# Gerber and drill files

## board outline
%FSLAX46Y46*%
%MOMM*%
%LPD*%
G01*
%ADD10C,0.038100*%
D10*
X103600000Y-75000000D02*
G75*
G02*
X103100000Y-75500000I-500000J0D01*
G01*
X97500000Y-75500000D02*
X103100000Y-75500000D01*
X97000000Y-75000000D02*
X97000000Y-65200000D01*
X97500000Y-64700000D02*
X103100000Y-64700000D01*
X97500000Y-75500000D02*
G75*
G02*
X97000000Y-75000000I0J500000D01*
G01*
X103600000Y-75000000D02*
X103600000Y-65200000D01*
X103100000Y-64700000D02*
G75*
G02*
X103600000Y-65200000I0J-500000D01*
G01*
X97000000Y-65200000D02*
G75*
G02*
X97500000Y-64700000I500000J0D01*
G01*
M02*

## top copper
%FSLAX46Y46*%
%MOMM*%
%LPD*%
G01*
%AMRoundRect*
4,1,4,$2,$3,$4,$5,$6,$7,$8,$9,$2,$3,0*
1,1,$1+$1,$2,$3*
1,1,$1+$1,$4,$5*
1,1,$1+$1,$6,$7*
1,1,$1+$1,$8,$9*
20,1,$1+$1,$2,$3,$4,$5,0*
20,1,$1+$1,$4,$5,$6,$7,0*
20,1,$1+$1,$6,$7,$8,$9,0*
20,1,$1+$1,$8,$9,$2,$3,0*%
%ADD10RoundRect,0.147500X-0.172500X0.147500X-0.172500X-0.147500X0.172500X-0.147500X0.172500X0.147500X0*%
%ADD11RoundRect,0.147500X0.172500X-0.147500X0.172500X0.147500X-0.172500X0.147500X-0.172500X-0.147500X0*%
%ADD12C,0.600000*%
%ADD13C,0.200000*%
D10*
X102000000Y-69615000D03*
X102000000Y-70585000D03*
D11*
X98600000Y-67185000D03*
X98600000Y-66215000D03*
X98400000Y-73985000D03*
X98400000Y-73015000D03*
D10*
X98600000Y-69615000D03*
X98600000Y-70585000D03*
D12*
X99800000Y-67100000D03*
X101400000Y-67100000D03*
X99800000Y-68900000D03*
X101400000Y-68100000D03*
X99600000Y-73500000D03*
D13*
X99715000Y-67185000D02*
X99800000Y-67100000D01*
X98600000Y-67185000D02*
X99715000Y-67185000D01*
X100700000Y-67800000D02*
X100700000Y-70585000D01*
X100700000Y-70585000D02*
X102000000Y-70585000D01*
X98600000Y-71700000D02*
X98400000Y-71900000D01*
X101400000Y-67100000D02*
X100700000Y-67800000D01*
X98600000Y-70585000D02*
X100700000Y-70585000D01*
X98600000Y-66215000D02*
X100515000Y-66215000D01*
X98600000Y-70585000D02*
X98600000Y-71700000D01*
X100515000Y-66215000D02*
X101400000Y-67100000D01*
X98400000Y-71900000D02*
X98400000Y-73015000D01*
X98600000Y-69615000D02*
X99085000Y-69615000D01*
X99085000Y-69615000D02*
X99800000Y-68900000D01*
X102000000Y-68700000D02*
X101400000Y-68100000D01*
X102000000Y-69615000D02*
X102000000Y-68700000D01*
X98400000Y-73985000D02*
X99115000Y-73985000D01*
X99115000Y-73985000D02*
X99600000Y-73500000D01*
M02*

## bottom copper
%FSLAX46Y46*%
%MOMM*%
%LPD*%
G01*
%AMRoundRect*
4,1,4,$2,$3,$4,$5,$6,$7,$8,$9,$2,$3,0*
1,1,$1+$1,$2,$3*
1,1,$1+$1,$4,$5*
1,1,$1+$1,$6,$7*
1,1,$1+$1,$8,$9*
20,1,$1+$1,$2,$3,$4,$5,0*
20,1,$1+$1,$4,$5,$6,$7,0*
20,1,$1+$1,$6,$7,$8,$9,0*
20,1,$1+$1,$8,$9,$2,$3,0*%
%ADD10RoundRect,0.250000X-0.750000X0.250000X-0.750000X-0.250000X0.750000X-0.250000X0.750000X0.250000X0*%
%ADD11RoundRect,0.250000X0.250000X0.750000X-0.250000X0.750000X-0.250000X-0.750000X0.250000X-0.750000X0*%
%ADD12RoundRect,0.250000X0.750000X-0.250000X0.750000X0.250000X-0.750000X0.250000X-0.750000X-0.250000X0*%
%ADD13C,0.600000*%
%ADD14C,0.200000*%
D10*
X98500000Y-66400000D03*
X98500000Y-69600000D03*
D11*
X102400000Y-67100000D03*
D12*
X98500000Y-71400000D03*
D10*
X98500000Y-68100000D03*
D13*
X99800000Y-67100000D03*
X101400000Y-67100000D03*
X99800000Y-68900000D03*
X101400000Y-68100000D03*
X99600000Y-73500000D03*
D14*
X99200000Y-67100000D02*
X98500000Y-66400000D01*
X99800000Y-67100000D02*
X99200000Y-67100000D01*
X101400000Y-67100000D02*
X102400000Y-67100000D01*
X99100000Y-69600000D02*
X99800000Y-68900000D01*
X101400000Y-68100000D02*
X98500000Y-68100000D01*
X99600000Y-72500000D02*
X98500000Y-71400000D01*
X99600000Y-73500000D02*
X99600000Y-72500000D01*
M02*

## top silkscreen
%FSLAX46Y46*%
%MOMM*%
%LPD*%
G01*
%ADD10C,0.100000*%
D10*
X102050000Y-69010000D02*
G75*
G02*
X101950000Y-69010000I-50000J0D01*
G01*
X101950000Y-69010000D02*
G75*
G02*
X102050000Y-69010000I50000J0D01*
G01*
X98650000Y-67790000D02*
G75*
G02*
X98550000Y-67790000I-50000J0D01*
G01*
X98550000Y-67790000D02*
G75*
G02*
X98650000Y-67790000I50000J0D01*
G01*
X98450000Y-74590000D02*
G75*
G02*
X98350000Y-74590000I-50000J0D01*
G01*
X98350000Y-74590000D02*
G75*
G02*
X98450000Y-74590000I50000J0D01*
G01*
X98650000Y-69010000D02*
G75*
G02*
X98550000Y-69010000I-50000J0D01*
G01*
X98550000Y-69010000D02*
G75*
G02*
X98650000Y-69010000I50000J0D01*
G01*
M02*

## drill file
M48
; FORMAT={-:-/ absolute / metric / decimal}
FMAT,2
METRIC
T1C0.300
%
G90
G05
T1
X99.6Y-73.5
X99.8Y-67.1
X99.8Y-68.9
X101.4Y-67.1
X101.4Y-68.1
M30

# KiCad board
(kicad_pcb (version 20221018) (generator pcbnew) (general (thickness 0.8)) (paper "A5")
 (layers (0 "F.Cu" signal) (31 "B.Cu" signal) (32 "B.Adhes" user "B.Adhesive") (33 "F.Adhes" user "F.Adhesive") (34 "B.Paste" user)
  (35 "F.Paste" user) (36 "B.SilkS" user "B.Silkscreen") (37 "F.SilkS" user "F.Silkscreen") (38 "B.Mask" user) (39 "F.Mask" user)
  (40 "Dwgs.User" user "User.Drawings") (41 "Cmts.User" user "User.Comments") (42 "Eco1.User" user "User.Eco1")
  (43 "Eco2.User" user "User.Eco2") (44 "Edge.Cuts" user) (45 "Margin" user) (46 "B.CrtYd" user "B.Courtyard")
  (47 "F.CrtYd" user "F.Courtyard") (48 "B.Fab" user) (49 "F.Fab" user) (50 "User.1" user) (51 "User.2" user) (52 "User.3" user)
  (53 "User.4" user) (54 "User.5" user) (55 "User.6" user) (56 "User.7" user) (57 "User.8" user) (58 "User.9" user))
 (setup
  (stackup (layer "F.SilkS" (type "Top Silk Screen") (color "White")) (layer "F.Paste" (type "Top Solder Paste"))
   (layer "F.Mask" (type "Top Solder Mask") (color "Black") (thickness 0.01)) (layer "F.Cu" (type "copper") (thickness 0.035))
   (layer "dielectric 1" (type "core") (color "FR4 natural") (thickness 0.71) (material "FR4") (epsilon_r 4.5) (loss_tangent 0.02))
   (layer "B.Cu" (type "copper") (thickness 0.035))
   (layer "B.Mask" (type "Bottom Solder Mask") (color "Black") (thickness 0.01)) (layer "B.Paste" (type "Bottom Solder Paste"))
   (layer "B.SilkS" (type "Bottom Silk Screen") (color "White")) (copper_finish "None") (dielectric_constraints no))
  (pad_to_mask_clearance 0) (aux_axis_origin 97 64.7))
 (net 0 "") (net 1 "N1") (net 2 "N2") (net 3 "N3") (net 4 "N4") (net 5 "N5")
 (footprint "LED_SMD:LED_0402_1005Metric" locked (layer "F.Cu") (at 102 70.1 -90)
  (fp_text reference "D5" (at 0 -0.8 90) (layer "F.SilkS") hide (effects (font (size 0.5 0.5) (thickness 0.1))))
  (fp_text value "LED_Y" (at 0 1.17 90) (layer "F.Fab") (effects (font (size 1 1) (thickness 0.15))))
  (fp_circle (center -1.09 0) (end -1.04 0) (stroke (width 0.1) (type solid)) (fill none) (layer "F.SilkS"))
  (pad "1" smd roundrect locked (at -0.485 0 270) (size 0.59 0.64) (layers "F.Cu" "F.Paste" "F.Mask") (roundrect_rratio 0.25) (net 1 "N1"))
  (pad "2" smd roundrect locked (at 0.485 0 270) (size 0.59 0.64) (layers "F.Cu" "F.Paste" "F.Mask") (roundrect_rratio 0.25) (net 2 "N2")))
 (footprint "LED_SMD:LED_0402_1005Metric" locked (layer "F.Cu") (at 98.6 66.7 90)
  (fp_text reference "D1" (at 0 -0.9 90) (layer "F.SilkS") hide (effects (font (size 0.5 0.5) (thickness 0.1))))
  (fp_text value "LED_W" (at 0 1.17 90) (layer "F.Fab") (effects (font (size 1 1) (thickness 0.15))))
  (fp_circle (center -1.09 0) (end -1.04 0) (stroke (width 0.1) (type solid)) (fill none) (layer "F.SilkS"))
  (pad "1" smd roundrect locked (at -0.485 0 90) (size 0.59 0.64) (layers "F.Cu" "F.Paste" "F.Mask") (roundrect_rratio 0.25) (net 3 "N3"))
  (pad "2" smd roundrect locked (at 0.485 0 90) (size 0.59 0.64) (layers "F.Cu" "F.Paste" "F.Mask") (roundrect_rratio 0.25) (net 2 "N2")))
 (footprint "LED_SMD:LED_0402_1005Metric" (layer "F.Cu") (at 98.4 73.5 90)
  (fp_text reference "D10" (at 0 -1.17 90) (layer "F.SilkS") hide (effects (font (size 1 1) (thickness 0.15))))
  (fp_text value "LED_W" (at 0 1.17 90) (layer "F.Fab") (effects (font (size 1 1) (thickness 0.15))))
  (fp_circle (center -1.09 0) (end -1.04 0) (stroke (width 0.1) (type solid)) (fill none) (layer "F.SilkS"))
  (pad "1" smd roundrect (at -0.485 0 90) (size 0.59 0.64) (layers "F.Cu" "F.Paste" "F.Mask") (roundrect_rratio 0.25) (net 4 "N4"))
  (pad "2" smd roundrect (at 0.485 0 90) (size 0.59 0.64) (layers "F.Cu" "F.Paste" "F.Mask") (roundrect_rratio 0.25) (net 2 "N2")))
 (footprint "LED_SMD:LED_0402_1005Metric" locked (layer "F.Cu") (at 98.6 70.1 -90)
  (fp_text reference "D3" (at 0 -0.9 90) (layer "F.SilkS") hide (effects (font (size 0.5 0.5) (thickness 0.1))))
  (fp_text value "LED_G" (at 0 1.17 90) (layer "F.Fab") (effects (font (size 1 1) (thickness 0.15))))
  (fp_circle (center -1.09 0) (end -1.04 0) (stroke (width 0.1) (type solid)) (fill none) (layer "F.SilkS"))
  (pad "1" smd roundrect locked (at -0.485 0 270) (size 0.59 0.64) (layers "F.Cu" "F.Paste" "F.Mask") (roundrect_rratio 0.25) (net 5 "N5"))
  (pad "2" smd roundrect locked (at 0.485 0 270) (size 0.59 0.64) (layers "F.Cu" "F.Paste" "F.Mask") (roundrect_rratio 0.25) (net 2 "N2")))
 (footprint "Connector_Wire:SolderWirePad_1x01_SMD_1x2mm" (layer "B.Cu") (at 98.5 66.4 -90)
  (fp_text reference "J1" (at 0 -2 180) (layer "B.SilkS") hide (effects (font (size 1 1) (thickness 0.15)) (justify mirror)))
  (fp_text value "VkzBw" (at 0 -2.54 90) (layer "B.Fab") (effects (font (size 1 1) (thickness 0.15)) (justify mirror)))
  (pad "1" smd roundrect (at 0 0 270) (size 1 2) (layers "B.Cu" "B.Paste" "B.Mask") (roundrect_rratio 0.25) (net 3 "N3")))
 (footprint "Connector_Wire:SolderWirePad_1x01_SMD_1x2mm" (layer "B.Cu") (at 98.5 69.6 -90)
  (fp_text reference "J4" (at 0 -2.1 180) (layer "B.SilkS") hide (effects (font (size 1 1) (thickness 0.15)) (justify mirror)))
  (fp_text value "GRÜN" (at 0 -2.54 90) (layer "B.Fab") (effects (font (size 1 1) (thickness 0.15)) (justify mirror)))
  (pad "1" smd roundrect (at 0 0 270) (size 1 2) (layers "B.Cu" "B.Paste" "B.Mask") (roundrect_rratio 0.25) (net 5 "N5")))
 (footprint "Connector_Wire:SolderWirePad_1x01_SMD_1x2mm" (layer "B.Cu") (at 102.4 67.1 180)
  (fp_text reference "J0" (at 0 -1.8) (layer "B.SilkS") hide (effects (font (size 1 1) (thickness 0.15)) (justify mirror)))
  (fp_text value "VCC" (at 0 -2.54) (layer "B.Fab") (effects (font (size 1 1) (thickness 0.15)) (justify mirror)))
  (pad "1" smd roundrect (at 0 0 180) (size 1 2) (layers "B.Cu" "B.Paste" "B.Mask") (roundrect_rratio 0.25) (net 2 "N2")))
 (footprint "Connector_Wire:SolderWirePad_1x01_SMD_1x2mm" (layer "B.Cu") (at 98.5 71.4 90)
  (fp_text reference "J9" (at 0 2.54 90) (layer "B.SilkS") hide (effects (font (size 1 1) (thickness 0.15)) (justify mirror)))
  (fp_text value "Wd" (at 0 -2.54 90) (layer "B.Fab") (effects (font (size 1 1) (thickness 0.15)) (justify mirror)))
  (pad "1" smd roundrect (at 0 0 90) (size 1 2) (layers "B.Cu" "B.Paste" "B.Mask") (roundrect_rratio 0.25) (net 4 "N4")))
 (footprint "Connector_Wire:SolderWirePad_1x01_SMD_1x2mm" (layer "B.Cu") (at 98.5 68.1 -90)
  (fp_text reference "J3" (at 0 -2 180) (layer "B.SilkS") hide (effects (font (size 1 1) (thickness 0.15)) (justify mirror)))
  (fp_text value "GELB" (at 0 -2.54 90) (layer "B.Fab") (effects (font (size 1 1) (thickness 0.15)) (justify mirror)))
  (pad "1" smd roundrect (at 0 0 270) (size 1 2) (layers "B.Cu" "B.Paste" "B.Mask") (roundrect_rratio 0.25) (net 1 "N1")))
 (gr_arc (start 103.6 75) (mid 103.453553 75.353553) (end 103.1 75.5) (stroke (width 0.0381) (type solid)) (layer "Edge.Cuts"))
 (gr_line (start 97.5 75.5) (end 103.1 75.5) (stroke (width 0.0381) (type solid)) (layer "Edge.Cuts"))
 (gr_line (start 97 75) (end 97 65.2) (stroke (width 0.0381) (type solid)) (layer "Edge.Cuts"))
 (gr_line (start 97.5 64.7) (end 103.1 64.7) (stroke (width 0.0381) (type solid)) (layer "Edge.Cuts"))
 (gr_arc (start 97.5 75.5) (mid 97.146447 75.353553) (end 97 75) (stroke (width 0.0381) (type solid)) (layer "Edge.Cuts"))
 (gr_line (start 103.6 75) (end 103.6 65.2) (stroke (width 0.0381) (type solid)) (layer "Edge.Cuts"))
 (gr_arc (start 103.1 64.7) (mid 103.453553 64.846447) (end 103.6 65.2) (stroke (width 0.0381) (type solid)) (layer "Edge.Cuts"))
 (gr_arc (start 97 65.2) (mid 97.146447 64.846447) (end 97.5 64.7) (stroke (width 0.0381) (type solid)) (layer "Edge.Cuts"))
 (segment (start 99.715 67.185) (end 99.8 67.1) (width 0.2) (layer "F.Cu") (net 3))
 (segment (start 98.6 67.185) (end 99.715 67.185) (width 0.2) (layer "F.Cu") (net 3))
 (via (at 99.8 67.1) (size 0.6) (drill 0.3) (layers "F.Cu" "B.Cu") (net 3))
 (segment (start 99.2 67.1) (end 98.5 66.4) (width 0.2) (layer "B.Cu") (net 3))
 (segment (start 99.8 67.1) (end 99.2 67.1) (width 0.2) (layer "B.Cu") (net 3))
 (segment (start 100.7 67.8) (end 100.7 70.585) (width 0.2) (layer "F.Cu") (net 2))
 (segment (start 100.7 70.585) (end 102 70.585) (width 0.2) (layer "F.Cu") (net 2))
 (segment (start 98.6 71.7) (end 98.4 71.9) (width 0.2) (layer "F.Cu") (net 2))
 (segment (start 101.4 67.1) (end 100.7 67.8) (width 0.2) (layer "F.Cu") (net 2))
 (segment (start 98.6 70.585) (end 100.7 70.585) (width 0.2) (layer "F.Cu") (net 2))
 (segment (start 98.6 66.215) (end 100.515 66.215) (width 0.2) (layer "F.Cu") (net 2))
 (segment (start 98.6 70.585) (end 98.6 71.7) (width 0.2) (layer "F.Cu") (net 2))
 (segment (start 100.515 66.215) (end 101.4 67.1) (width 0.2) (layer "F.Cu") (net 2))
 (segment (start 98.4 71.9) (end 98.4 73.015) (width 0.2) (layer "F.Cu") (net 2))
 (via (at 101.4 67.1) (size 0.6) (drill 0.3) (layers "F.Cu" "B.Cu") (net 2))
 (segment (start 101.4 67.1) (end 102.4 67.1) (width 0.2) (layer "B.Cu") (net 2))
 (segment (start 98.6 69.615) (end 99.085 69.615) (width 0.2) (layer "F.Cu") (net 5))
 (segment (start 99.085 69.615) (end 99.8 68.9) (width 0.2) (layer "F.Cu") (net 5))
 (via (at 99.8 68.9) (size 0.6) (drill 0.3) (layers "F.Cu" "B.Cu") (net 5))
 (segment (start 99.1 69.6) (end 99.8 68.9) (width 0.2) (layer "B.Cu") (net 5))
 (segment (start 102 68.7) (end 101.4 68.1) (width 0.2) (layer "F.Cu") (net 1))
 (segment (start 102 69.615) (end 102 68.7) (width 0.2) (layer "F.Cu") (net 1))
 (via (at 101.4 68.1) (size 0.6) (drill 0.3) (layers "F.Cu" "B.Cu") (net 1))
 (segment (start 101.4 68.1) (end 98.5 68.1) (width 0.2) (layer "B.Cu") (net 1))
 (segment (start 98.4 73.985) (end 99.115 73.985) (width 0.2) (layer "F.Cu") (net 4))
 (segment (start 99.115 73.985) (end 99.6 73.5) (width 0.2) (layer "F.Cu") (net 4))
 (via (at 99.6 73.5) (size 0.6) (drill 0.3) (layers "F.Cu" "B.Cu") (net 4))
 (segment (start 99.6 72.5) (end 98.5 71.4) (width 0.2) (layer "B.Cu") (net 4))
 (segment (start 99.6 73.5) (end 99.6 72.5) (width 0.2) (layer "B.Cu") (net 4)))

